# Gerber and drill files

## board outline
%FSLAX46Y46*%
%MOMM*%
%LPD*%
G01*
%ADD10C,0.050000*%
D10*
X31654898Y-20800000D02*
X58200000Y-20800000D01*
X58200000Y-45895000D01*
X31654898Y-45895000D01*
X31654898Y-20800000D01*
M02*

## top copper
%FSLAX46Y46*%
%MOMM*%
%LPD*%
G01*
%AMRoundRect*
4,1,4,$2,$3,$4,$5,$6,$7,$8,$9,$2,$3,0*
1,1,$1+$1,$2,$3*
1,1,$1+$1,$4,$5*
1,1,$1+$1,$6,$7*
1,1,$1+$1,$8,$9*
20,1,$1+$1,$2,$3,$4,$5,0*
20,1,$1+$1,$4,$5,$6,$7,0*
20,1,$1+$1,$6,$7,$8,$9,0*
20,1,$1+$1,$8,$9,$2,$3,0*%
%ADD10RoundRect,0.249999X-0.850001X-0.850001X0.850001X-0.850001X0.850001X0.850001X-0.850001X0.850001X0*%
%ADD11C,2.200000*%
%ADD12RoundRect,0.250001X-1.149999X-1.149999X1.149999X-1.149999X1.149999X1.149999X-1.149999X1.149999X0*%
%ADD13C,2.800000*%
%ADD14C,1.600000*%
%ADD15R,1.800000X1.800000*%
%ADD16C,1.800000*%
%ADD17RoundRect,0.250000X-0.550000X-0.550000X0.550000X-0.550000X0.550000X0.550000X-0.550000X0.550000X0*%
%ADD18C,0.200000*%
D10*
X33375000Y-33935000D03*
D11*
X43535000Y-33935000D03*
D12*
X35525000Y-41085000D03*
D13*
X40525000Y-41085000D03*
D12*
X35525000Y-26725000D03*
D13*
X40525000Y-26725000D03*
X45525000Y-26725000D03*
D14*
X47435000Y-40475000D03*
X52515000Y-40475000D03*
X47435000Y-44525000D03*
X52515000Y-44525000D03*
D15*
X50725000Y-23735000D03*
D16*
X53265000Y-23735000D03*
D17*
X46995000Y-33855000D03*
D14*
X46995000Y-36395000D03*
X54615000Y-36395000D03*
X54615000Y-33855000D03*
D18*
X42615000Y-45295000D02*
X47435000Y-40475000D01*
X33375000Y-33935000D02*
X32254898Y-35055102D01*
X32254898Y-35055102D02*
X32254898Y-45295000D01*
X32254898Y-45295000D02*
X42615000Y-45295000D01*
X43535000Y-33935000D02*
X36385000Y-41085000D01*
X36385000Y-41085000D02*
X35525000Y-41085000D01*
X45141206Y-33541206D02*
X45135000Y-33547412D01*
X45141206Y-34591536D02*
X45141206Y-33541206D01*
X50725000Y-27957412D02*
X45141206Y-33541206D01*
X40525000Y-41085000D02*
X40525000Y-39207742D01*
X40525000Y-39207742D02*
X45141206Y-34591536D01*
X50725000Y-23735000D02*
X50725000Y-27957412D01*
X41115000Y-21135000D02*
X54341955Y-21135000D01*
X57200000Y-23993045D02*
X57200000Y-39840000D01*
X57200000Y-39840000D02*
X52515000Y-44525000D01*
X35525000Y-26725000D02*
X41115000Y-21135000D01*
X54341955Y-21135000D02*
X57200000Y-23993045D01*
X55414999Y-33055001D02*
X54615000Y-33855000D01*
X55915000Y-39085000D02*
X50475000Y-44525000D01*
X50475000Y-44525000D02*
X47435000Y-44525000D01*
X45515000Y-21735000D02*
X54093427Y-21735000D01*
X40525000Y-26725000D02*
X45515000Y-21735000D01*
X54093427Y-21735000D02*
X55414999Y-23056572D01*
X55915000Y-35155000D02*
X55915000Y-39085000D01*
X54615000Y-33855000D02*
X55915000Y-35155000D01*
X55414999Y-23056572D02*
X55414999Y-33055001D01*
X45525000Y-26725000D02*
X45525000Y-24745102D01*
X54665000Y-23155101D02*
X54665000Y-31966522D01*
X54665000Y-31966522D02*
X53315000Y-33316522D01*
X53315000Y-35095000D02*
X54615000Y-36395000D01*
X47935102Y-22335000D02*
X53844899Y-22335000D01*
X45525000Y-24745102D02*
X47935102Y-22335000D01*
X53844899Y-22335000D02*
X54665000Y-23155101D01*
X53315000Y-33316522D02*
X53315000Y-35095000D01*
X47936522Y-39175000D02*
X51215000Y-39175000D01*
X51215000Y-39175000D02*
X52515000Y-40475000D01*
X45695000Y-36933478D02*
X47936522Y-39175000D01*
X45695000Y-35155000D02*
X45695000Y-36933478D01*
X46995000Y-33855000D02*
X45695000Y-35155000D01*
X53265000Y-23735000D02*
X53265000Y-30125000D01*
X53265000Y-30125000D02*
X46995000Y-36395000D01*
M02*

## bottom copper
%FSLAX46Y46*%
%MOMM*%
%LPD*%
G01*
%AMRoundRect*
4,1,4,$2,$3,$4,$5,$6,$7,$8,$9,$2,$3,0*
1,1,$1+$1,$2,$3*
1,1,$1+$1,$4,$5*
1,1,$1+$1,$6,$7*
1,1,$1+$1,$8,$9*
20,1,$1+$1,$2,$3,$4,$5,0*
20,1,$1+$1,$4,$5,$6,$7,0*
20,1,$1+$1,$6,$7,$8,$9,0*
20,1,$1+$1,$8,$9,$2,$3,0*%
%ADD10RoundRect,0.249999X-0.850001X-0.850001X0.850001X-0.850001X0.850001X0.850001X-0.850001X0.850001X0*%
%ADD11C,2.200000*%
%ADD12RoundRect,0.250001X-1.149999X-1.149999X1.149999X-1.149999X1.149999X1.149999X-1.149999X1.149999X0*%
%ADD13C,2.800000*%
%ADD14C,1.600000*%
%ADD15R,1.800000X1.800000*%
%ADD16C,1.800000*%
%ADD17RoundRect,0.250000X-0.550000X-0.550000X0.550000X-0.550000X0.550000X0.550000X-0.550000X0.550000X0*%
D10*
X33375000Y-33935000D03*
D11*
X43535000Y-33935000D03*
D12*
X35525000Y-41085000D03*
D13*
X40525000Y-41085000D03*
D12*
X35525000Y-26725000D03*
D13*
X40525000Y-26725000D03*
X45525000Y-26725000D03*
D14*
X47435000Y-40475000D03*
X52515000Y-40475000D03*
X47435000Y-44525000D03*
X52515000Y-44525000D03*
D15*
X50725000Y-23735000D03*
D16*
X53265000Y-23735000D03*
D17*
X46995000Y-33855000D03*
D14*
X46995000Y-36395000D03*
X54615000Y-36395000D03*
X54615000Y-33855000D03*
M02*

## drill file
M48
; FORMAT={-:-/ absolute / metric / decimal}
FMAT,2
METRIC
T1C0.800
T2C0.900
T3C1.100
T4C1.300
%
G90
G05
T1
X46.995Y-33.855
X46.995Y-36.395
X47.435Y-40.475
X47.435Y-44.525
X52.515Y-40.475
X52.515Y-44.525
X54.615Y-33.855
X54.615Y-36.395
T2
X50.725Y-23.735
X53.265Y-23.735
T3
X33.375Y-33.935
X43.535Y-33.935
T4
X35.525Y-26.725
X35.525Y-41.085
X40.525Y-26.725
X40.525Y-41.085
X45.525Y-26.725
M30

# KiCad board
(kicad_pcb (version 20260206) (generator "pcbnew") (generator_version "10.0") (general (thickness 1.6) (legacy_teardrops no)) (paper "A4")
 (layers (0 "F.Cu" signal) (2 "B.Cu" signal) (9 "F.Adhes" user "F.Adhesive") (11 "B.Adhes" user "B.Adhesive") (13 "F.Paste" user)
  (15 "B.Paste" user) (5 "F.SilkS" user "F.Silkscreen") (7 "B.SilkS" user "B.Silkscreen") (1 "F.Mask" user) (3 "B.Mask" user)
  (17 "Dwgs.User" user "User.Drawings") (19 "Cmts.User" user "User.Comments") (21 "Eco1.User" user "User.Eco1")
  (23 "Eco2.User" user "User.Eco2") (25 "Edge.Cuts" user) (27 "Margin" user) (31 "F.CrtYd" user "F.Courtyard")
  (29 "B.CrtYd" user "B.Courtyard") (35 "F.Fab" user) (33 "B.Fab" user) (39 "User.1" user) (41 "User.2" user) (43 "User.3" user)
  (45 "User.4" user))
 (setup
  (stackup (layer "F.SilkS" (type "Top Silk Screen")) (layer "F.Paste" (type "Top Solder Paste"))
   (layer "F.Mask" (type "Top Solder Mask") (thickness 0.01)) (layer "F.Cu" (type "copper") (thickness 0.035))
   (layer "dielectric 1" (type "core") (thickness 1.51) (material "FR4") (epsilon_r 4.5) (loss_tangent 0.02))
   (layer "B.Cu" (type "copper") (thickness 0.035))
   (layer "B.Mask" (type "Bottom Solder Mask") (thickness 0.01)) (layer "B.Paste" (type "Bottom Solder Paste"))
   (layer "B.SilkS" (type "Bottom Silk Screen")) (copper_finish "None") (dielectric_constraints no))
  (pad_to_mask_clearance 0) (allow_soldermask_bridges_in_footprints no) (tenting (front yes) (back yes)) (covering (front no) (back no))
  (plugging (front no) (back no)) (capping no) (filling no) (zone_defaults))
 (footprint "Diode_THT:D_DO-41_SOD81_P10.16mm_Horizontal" (layer "F.Cu") (at 33.375 33.935)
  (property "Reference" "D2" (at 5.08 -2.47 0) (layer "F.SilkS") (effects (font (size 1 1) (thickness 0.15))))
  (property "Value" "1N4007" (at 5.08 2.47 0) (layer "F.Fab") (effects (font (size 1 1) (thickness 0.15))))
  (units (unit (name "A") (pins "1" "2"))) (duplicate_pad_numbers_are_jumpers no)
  (pad "1" thru_hole roundrect (at 0 0) (size 2.2 2.2) (drill 1.1) (layers "*.Cu" "*.Mask") (remove_unused_layers no)
   (roundrect_rratio 0.113636) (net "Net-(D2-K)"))
  (pad "2" thru_hole circle (at 10.16 0) (size 2.2 2.2) (drill 1.1) (layers "*.Cu" "*.Mask") (remove_unused_layers no) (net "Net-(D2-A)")))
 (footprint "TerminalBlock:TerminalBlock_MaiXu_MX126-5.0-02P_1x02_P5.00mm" (layer "F.Cu") (at 35.525 41.085)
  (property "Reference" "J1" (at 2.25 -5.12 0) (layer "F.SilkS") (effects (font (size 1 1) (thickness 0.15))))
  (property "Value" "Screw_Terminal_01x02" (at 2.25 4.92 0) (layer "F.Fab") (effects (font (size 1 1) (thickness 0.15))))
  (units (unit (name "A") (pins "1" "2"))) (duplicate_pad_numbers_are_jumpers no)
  (pad "1" thru_hole roundrect (at 0 0) (size 2.8 2.8) (drill 1.3) (layers "*.Cu" "*.Mask") (remove_unused_layers no)
   (roundrect_rratio 0.089286) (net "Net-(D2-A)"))
  (pad "2" thru_hole circle (at 5 0) (size 2.8 2.8) (drill 1.3) (layers "*.Cu" "*.Mask") (remove_unused_layers no) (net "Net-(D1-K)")))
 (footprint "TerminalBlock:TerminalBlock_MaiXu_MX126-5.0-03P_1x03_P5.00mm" (layer "F.Cu") (at 35.525 26.725)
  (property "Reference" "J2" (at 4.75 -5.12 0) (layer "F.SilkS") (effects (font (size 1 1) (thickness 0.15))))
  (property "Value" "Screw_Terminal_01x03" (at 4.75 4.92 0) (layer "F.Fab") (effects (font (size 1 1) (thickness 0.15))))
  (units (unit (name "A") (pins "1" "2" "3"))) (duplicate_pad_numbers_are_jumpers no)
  (pad "1" thru_hole roundrect (at 0 0) (size 2.8 2.8) (drill 1.3) (layers "*.Cu" "*.Mask") (remove_unused_layers no)
   (roundrect_rratio 0.089286) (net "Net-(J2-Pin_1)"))
  (pad "2" thru_hole circle (at 5 0) (size 2.8 2.8) (drill 1.3) (layers "*.Cu" "*.Mask") (remove_unused_layers no) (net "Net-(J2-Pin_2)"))
  (pad "3" thru_hole circle (at 10 0) (size 2.8 2.8) (drill 1.3) (layers "*.Cu" "*.Mask") (remove_unused_layers no) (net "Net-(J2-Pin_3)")))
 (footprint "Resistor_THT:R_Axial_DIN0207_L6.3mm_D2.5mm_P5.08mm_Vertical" (layer "F.Cu") (at 47.435 40.475)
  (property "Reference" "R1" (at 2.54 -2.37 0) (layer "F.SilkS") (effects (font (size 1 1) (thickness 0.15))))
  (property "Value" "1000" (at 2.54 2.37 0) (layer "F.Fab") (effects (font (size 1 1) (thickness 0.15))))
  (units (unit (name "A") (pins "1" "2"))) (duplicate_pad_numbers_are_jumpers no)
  (pad "1" thru_hole circle (at 0 0) (size 1.6 1.6) (drill 0.8) (layers "*.Cu" "*.Mask") (remove_unused_layers no) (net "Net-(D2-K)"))
  (pad "2" thru_hole circle (at 5.08 0) (size 1.6 1.6) (drill 0.8) (layers "*.Cu" "*.Mask") (remove_unused_layers no) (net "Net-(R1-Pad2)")))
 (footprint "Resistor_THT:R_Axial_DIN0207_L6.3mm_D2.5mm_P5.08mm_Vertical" (layer "F.Cu") (at 47.435 44.525)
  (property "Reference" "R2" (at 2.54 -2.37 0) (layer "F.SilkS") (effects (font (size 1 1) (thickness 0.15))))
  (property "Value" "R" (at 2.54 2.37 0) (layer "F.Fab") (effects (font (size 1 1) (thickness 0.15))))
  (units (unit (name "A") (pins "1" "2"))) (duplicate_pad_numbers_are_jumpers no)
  (pad "1" thru_hole circle (at 0 0) (size 1.6 1.6) (drill 0.8) (layers "*.Cu" "*.Mask") (remove_unused_layers no) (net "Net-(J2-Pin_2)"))
  (pad "2" thru_hole circle (at 5.08 0) (size 1.6 1.6) (drill 0.8) (layers "*.Cu" "*.Mask") (remove_unused_layers no) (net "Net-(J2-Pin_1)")))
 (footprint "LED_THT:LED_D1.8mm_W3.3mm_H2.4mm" (layer "F.Cu") (at 50.725 23.735)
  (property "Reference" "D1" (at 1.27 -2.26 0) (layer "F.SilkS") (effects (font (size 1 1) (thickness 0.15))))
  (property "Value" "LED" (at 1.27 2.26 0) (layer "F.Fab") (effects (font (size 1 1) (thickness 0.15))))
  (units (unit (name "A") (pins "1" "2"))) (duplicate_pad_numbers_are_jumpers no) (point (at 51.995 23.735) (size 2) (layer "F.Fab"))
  (pad "1" thru_hole rect (at 0 0) (size 1.8 1.8) (drill 0.9) (layers "*.Cu" "*.Mask") (remove_unused_layers no) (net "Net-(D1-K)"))
  (pad "2" thru_hole circle (at 2.54 0) (size 1.8 1.8) (drill 0.9) (layers "*.Cu" "*.Mask") (remove_unused_layers no) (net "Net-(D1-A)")))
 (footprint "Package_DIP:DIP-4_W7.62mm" (layer "F.Cu") (at 46.995 33.855)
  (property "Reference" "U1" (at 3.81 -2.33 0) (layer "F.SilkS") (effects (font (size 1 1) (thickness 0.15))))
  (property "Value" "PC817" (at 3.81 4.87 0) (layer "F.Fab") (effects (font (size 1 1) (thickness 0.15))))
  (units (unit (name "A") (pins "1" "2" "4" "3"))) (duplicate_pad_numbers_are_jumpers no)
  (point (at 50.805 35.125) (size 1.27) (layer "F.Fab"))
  (pad "1" thru_hole roundrect (at 0 0) (size 1.6 1.6) (drill 0.8) (layers "*.Cu" "*.Mask") (remove_unused_layers no)
   (roundrect_rratio 0.15625) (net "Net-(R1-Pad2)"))
  (pad "2" thru_hole circle (at 0 2.54) (size 1.6 1.6) (drill 0.8) (layers "*.Cu" "*.Mask") (remove_unused_layers no) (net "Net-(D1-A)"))
  (pad "3" thru_hole circle (at 7.62 2.54) (size 1.6 1.6) (drill 0.8) (layers "*.Cu" "*.Mask") (remove_unused_layers no)
   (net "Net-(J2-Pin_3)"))
  (pad "4" thru_hole circle (at 7.62 0) (size 1.6 1.6) (drill 0.8) (layers "*.Cu" "*.Mask") (remove_unused_layers no) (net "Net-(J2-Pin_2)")))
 (gr_rect (start 31.654898 20.8) (end 58.2 45.895) (stroke (width 0.05) (type default)) (fill no) (layer "Edge.Cuts"))
 (segment (start 42.615 45.295) (end 47.435 40.475) (width 0.2) (layer "F.Cu") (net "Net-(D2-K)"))
 (segment (start 33.375 33.935) (end 32.254898 35.055102) (width 0.2) (layer "F.Cu") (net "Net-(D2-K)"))
 (segment (start 32.254898 35.055102) (end 32.254898 45.295) (width 0.2) (layer "F.Cu") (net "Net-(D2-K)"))
 (segment (start 32.254898 45.295) (end 42.615 45.295) (width 0.2) (layer "F.Cu") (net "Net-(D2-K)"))
 (segment (start 43.535 33.935) (end 36.385 41.085) (width 0.2) (layer "F.Cu") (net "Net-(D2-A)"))
 (segment (start 36.385 41.085) (end 35.525 41.085) (width 0.2) (layer "F.Cu") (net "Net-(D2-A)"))
 (segment (start 45.141206 33.541206) (end 45.135 33.547412) (width 0.2) (layer "F.Cu") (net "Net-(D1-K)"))
 (segment (start 45.141206 34.591536) (end 45.141206 33.541206) (width 0.2) (layer "F.Cu") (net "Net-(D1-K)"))
 (segment (start 50.725 27.957412) (end 45.141206 33.541206) (width 0.2) (layer "F.Cu") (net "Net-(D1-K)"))
 (segment (start 40.525 41.085) (end 40.525 39.207742) (width 0.2) (layer "F.Cu") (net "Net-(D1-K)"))
 (segment (start 40.525 39.207742) (end 45.141206 34.591536) (width 0.2) (layer "F.Cu") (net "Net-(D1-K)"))
 (segment (start 50.725 23.735) (end 50.725 27.957412) (width 0.2) (layer "F.Cu") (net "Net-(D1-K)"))
 (segment (start 41.115 21.135) (end 54.341955 21.135) (width 0.2) (layer "F.Cu") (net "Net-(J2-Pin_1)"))
 (segment (start 57.2 23.993045) (end 57.2 39.84) (width 0.2) (layer "F.Cu") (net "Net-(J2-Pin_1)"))
 (segment (start 57.2 39.84) (end 52.515 44.525) (width 0.2) (layer "F.Cu") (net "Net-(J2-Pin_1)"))
 (segment (start 35.525 26.725) (end 41.115 21.135) (width 0.2) (layer "F.Cu") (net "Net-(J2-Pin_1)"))
 (segment (start 54.341955 21.135) (end 57.2 23.993045) (width 0.2) (layer "F.Cu") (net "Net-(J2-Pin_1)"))
 (segment (start 55.414999 33.055001) (end 54.615 33.855) (width 0.2) (layer "F.Cu") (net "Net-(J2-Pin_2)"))
 (segment (start 55.915 39.085) (end 50.475 44.525) (width 0.2) (layer "F.Cu") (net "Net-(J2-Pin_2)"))
 (segment (start 50.475 44.525) (end 47.435 44.525) (width 0.2) (layer "F.Cu") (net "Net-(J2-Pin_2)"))
 (segment (start 45.515 21.735) (end 54.093427 21.735) (width 0.2) (layer "F.Cu") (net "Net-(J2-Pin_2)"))
 (segment (start 40.525 26.725) (end 45.515 21.735) (width 0.2) (layer "F.Cu") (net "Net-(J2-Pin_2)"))
 (segment (start 54.093427 21.735) (end 55.414999 23.056572) (width 0.2) (layer "F.Cu") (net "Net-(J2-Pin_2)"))
 (segment (start 55.915 35.155) (end 55.915 39.085) (width 0.2) (layer "F.Cu") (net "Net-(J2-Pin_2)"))
 (segment (start 54.615 33.855) (end 55.915 35.155) (width 0.2) (layer "F.Cu") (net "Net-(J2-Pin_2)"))
 (segment (start 55.414999 23.056572) (end 55.414999 33.055001) (width 0.2) (layer "F.Cu") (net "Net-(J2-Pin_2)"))
 (segment (start 45.525 26.725) (end 45.525 24.745102) (width 0.2) (layer "F.Cu") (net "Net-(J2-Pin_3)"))
 (segment (start 54.665 23.155101) (end 54.665 31.966522) (width 0.2) (layer "F.Cu") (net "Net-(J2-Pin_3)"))
 (segment (start 54.665 31.966522) (end 53.315 33.316522) (width 0.2) (layer "F.Cu") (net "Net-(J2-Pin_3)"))
 (segment (start 53.315 35.095) (end 54.615 36.395) (width 0.2) (layer "F.Cu") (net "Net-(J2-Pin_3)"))
 (segment (start 47.935102 22.335) (end 53.844899 22.335) (width 0.2) (layer "F.Cu") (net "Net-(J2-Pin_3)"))
 (segment (start 45.525 24.745102) (end 47.935102 22.335) (width 0.2) (layer "F.Cu") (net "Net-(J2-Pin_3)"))
 (segment (start 53.844899 22.335) (end 54.665 23.155101) (width 0.2) (layer "F.Cu") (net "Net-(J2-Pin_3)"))
 (segment (start 53.315 33.316522) (end 53.315 35.095) (width 0.2) (layer "F.Cu") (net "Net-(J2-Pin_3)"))
 (segment (start 47.936522 39.175) (end 51.215 39.175) (width 0.2) (layer "F.Cu") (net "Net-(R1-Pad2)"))
 (segment (start 51.215 39.175) (end 52.515 40.475) (width 0.2) (layer "F.Cu") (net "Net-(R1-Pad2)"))
 (segment (start 45.695 36.933478) (end 47.936522 39.175) (width 0.2) (layer "F.Cu") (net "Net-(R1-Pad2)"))
 (segment (start 45.695 35.155) (end 45.695 36.933478) (width 0.2) (layer "F.Cu") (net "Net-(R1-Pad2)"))
 (segment (start 46.995 33.855) (end 45.695 35.155) (width 0.2) (layer "F.Cu") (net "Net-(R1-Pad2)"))
 (segment (start 53.265 23.735) (end 53.265 30.125) (width 0.2) (layer "F.Cu") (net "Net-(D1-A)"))
 (segment (start 53.265 30.125) (end 46.995 36.395) (width 0.2) (layer "F.Cu") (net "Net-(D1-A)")))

